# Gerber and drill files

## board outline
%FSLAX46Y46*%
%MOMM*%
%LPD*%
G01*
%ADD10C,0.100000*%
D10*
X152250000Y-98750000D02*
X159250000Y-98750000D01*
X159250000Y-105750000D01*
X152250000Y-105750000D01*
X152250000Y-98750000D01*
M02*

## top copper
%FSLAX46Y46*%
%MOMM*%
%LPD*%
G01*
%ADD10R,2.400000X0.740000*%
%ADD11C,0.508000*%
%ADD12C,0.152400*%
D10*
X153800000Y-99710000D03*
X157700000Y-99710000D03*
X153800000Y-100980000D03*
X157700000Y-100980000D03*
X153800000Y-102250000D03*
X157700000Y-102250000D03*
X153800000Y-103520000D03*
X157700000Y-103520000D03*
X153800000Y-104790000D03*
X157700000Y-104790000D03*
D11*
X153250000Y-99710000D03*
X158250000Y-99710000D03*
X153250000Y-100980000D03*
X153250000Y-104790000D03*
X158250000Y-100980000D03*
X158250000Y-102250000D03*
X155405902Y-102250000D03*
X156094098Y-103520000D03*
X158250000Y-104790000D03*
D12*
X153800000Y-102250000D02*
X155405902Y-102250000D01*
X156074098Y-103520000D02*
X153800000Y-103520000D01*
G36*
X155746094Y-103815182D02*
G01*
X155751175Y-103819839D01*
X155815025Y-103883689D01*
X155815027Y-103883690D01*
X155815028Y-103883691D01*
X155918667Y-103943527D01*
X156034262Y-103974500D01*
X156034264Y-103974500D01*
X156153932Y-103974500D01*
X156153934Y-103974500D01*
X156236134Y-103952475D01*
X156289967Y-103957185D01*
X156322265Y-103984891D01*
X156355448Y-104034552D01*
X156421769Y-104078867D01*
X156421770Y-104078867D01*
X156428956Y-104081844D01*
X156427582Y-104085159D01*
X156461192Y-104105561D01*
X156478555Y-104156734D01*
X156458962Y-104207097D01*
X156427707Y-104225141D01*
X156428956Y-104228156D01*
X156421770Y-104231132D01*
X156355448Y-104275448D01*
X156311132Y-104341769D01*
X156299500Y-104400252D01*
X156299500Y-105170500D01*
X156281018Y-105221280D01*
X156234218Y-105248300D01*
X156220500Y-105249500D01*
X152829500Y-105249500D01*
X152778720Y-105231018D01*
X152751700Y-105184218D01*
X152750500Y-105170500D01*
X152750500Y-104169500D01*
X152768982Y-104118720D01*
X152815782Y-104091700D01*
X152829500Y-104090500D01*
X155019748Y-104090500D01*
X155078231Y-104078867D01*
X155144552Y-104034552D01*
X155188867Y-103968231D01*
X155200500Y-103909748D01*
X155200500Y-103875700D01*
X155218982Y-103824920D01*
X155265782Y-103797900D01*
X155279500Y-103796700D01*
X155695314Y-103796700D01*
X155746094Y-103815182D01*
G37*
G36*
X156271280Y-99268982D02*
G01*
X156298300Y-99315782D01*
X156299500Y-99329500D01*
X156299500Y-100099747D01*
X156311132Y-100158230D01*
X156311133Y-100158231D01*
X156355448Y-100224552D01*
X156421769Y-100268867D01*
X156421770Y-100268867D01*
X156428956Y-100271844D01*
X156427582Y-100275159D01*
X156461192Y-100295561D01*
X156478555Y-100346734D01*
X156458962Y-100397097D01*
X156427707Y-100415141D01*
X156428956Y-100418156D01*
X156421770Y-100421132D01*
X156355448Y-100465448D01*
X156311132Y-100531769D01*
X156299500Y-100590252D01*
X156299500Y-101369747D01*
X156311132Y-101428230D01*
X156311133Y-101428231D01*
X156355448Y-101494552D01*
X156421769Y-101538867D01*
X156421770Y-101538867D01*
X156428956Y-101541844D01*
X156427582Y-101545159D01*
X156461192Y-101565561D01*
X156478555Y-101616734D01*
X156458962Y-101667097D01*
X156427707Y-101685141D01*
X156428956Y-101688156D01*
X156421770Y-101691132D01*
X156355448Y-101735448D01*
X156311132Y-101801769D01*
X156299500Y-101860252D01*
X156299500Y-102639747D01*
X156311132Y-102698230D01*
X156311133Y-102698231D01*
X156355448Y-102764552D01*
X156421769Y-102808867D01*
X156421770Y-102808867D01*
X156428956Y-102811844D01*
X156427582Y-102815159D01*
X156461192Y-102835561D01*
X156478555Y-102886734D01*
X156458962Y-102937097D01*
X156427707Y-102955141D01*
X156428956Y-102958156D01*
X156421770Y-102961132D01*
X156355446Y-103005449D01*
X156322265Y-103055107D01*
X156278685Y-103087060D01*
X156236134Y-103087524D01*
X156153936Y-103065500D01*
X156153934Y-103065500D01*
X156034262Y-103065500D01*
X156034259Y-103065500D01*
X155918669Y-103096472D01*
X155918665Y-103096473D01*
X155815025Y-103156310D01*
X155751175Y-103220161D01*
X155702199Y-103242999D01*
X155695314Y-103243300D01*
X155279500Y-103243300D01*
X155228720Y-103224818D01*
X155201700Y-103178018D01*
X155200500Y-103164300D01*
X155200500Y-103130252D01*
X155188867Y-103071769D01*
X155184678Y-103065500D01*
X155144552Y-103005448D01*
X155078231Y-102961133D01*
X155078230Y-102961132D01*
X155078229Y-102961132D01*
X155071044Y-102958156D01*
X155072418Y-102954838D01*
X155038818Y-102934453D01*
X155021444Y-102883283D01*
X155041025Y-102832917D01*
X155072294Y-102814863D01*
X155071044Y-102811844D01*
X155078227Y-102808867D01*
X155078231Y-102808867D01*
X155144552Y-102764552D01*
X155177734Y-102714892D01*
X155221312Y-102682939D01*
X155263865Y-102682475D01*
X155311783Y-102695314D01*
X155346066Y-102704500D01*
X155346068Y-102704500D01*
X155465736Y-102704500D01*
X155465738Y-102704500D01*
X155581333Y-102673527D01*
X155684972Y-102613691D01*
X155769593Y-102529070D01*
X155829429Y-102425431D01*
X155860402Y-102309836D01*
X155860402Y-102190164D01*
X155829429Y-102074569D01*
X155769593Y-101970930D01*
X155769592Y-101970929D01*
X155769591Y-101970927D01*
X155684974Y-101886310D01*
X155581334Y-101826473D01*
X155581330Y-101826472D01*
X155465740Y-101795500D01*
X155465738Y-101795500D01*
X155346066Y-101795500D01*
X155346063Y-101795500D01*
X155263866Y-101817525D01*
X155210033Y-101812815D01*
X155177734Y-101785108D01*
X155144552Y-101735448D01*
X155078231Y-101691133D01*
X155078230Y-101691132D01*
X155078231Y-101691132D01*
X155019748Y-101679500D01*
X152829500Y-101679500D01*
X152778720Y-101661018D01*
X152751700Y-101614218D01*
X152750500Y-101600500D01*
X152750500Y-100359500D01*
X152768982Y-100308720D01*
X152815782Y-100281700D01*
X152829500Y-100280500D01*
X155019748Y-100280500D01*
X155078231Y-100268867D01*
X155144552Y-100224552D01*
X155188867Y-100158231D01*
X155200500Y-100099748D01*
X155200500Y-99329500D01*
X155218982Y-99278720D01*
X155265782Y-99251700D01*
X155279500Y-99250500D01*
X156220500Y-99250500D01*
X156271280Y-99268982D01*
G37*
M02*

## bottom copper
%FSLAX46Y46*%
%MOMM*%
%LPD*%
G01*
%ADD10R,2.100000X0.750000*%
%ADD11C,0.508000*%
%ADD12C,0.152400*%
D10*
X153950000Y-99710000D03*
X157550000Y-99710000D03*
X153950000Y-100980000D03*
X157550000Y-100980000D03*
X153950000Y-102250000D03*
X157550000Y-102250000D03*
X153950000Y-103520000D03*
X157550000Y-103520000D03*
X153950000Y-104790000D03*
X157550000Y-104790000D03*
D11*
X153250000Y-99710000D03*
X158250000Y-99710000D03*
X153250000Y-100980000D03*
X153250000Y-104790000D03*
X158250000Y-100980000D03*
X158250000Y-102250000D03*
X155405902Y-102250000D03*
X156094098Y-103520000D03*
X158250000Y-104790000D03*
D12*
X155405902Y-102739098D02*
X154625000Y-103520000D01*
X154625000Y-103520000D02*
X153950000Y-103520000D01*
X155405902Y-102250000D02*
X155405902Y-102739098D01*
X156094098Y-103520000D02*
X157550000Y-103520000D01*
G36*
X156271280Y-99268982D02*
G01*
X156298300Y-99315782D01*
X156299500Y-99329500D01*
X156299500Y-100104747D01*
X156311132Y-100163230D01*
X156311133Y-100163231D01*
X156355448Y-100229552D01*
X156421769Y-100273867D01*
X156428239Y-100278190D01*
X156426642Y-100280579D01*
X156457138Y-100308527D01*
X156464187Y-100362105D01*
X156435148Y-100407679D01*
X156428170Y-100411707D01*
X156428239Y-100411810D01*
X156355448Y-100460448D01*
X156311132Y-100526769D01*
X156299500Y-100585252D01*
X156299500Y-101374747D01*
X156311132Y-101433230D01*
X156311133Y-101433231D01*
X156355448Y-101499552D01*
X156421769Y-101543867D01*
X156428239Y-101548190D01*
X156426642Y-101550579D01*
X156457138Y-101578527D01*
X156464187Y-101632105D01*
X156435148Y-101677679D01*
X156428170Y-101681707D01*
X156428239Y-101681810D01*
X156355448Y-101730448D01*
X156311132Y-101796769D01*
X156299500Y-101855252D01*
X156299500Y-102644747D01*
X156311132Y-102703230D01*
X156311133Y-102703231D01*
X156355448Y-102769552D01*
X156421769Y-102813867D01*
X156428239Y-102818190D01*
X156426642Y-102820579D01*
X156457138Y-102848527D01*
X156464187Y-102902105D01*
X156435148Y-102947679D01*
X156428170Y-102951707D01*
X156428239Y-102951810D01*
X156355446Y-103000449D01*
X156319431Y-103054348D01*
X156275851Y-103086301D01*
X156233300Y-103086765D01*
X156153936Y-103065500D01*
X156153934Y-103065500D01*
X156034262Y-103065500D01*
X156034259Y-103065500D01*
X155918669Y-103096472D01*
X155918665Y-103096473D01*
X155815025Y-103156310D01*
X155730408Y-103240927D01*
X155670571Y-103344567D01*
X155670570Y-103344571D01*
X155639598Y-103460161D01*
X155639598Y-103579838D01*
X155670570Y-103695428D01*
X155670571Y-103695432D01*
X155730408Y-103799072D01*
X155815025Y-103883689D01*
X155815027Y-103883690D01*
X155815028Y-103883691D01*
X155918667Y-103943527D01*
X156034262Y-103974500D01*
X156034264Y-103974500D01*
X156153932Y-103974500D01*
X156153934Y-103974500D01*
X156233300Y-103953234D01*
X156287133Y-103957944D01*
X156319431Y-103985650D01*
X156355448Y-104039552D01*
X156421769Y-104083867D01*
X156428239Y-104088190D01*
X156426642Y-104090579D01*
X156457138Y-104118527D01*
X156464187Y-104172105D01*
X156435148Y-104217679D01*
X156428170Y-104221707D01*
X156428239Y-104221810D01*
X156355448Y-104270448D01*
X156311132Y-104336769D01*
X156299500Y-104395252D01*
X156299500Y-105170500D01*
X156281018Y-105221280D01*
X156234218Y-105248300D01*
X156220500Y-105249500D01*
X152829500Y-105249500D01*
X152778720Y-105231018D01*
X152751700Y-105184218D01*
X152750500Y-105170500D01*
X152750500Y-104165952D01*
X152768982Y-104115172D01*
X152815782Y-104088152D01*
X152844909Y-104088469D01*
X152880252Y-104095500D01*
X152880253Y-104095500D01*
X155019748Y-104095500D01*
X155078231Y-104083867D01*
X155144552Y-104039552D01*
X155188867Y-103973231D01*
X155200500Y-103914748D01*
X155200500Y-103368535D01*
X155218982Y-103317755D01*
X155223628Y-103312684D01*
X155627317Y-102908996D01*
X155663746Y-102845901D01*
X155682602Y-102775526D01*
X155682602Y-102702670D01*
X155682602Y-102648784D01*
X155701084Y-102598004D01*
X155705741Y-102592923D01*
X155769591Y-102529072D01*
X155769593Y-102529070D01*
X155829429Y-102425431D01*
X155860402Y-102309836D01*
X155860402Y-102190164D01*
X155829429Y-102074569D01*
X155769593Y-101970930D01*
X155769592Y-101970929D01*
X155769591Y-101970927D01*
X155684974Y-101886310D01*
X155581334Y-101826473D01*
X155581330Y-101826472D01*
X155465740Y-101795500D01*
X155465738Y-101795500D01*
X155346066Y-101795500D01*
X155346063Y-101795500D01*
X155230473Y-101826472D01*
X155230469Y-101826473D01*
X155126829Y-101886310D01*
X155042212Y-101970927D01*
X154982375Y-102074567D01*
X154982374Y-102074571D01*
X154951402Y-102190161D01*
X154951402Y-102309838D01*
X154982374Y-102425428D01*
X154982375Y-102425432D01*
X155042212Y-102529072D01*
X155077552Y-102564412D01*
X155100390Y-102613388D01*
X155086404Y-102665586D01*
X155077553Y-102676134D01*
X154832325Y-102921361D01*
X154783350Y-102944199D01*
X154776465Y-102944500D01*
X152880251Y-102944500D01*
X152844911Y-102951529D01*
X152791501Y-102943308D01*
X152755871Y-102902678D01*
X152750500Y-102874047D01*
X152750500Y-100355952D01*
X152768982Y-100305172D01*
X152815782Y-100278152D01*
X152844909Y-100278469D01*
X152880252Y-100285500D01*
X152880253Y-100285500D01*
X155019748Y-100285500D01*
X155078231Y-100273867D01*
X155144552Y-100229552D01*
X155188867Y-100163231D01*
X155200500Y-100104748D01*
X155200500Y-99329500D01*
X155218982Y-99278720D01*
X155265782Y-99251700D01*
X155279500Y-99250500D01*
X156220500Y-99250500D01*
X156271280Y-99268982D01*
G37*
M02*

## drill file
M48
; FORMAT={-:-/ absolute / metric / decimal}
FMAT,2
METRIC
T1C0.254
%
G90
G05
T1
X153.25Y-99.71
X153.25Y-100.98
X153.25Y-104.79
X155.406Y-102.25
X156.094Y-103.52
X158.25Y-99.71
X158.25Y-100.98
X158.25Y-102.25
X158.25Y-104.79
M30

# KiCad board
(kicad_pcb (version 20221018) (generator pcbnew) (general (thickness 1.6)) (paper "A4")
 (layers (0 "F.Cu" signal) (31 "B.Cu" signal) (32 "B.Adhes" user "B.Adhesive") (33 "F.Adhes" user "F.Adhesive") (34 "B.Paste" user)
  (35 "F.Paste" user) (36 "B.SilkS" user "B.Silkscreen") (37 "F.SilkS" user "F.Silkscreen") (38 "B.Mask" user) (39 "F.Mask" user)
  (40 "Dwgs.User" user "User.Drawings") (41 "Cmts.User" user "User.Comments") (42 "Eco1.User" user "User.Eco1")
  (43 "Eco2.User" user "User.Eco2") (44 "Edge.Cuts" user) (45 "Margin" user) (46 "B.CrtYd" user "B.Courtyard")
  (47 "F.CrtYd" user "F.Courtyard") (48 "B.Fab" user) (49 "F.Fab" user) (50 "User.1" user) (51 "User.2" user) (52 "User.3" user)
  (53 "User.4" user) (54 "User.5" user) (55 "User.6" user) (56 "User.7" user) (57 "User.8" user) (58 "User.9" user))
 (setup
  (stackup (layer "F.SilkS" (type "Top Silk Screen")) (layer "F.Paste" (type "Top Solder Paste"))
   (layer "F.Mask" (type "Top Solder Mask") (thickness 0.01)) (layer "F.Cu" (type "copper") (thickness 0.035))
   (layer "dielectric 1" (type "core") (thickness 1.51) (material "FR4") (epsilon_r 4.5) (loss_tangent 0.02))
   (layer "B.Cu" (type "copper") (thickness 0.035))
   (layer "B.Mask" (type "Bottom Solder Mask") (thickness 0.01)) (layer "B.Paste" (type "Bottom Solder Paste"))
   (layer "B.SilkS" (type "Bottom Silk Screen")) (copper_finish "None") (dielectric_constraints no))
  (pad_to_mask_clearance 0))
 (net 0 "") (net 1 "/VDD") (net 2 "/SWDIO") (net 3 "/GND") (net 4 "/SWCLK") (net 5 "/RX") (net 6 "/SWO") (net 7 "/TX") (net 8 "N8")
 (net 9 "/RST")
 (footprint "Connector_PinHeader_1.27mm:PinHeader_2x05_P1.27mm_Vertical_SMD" (layer "F.Cu") (at 155.75 102.25)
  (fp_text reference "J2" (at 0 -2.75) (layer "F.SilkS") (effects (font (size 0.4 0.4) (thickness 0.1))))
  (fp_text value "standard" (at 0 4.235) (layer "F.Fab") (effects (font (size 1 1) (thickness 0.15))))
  (pad "1" smd rect (at -1.95 -2.54) (size 2.4 0.74) (layers "F.Cu" "F.Paste" "F.Mask") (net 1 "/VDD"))
  (pad "2" smd rect (at 1.95 -2.54) (size 2.4 0.74) (layers "F.Cu" "F.Paste" "F.Mask") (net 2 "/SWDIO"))
  (pad "3" smd rect (at -1.95 -1.27) (size 2.4 0.74) (layers "F.Cu" "F.Paste" "F.Mask") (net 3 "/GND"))
  (pad "4" smd rect (at 1.95 -1.27) (size 2.4 0.74) (layers "F.Cu" "F.Paste" "F.Mask") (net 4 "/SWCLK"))
  (pad "5" smd rect (at -1.95 0) (size 2.4 0.74) (layers "F.Cu" "F.Paste" "F.Mask") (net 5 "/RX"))
  (pad "6" smd rect (at 1.95 0) (size 2.4 0.74) (layers "F.Cu" "F.Paste" "F.Mask") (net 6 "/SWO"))
  (pad "7" smd rect (at -1.95 1.27) (size 2.4 0.74) (layers "F.Cu" "F.Paste" "F.Mask") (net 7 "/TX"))
  (pad "8" smd rect (at 1.95 1.27) (size 2.4 0.74) (layers "F.Cu" "F.Paste" "F.Mask") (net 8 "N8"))
  (pad "9" smd rect (at -1.95 2.54) (size 2.4 0.74) (layers "F.Cu" "F.Paste" "F.Mask") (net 3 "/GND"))
  (pad "10" smd rect (at 1.95 2.54) (size 2.4 0.74) (layers "F.Cu" "F.Paste" "F.Mask") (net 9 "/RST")))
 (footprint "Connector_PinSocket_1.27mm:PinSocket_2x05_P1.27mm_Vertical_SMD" (layer "B.Cu") (at 155.75 102.25 180)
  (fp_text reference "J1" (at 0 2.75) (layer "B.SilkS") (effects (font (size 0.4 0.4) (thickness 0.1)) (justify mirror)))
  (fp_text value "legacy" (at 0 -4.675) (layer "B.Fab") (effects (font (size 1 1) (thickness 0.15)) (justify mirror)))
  (pad "1" smd rect (at 1.8 2.54 180) (size 2.1 0.75) (layers "B.Cu" "B.Paste" "B.Mask") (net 1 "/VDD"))
  (pad "2" smd rect (at -1.8 2.54 180) (size 2.1 0.75) (layers "B.Cu" "B.Paste" "B.Mask") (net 2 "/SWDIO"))
  (pad "3" smd rect (at 1.8 1.27 180) (size 2.1 0.75) (layers "B.Cu" "B.Paste" "B.Mask") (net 3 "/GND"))
  (pad "4" smd rect (at -1.8 1.27 180) (size 2.1 0.75) (layers "B.Cu" "B.Paste" "B.Mask") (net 4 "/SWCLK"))
  (pad "5" smd rect (at 1.8 0 180) (size 2.1 0.75) (layers "B.Cu" "B.Paste" "B.Mask") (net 3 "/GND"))
  (pad "6" smd rect (at -1.8 0 180) (size 2.1 0.75) (layers "B.Cu" "B.Paste" "B.Mask") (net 6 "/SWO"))
  (pad "7" smd rect (at 1.8 -1.27 180) (size 2.1 0.75) (layers "B.Cu" "B.Paste" "B.Mask") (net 5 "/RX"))
  (pad "8" smd rect (at -1.8 -1.27 180) (size 2.1 0.75) (layers "B.Cu" "B.Paste" "B.Mask") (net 7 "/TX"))
  (pad "9" smd rect (at 1.8 -2.54 180) (size 2.1 0.75) (layers "B.Cu" "B.Paste" "B.Mask") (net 3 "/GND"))
  (pad "10" smd rect (at -1.8 -2.54 180) (size 2.1 0.75) (layers "B.Cu" "B.Paste" "B.Mask") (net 9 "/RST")))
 (gr_rect (start 152.25 98.75) (end 159.25 105.75) (stroke (width 0.1) (type solid)) (fill none) (layer "Edge.Cuts"))
 (via (at 153.25 99.71) (size 0.508) (drill 0.254) (layers "F.Cu" "B.Cu") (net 1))
 (via (at 158.25 99.71) (size 0.508) (drill 0.254) (layers "F.Cu" "B.Cu") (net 2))
 (via (at 153.25 100.98) (size 0.508) (drill 0.254) (layers "F.Cu" "B.Cu") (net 3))
 (via (at 153.25 104.79) (size 0.508) (drill 0.254) (layers "F.Cu" "B.Cu") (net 3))
 (via (at 158.25 100.98) (size 0.508) (drill 0.254) (layers "F.Cu" "B.Cu") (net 4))
 (via (at 158.25 102.25) (size 0.508) (drill 0.254) (layers "F.Cu" "B.Cu") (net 6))
 (segment (start 153.8 102.25) (end 155.405902 102.25) (width 0.1524) (layer "F.Cu") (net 5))
 (via (at 155.405902 102.25) (size 0.508) (drill 0.254) (layers "F.Cu" "B.Cu") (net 5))
 (segment (start 155.405902 102.739098) (end 154.625 103.52) (width 0.1524) (layer "B.Cu") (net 5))
 (segment (start 154.625 103.52) (end 153.95 103.52) (width 0.1524) (layer "B.Cu") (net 5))
 (segment (start 155.405902 102.25) (end 155.405902 102.739098) (width 0.1524) (layer "B.Cu") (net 5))
 (segment (start 156.074098 103.52) (end 153.8 103.52) (width 0.1524) (layer "F.Cu") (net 7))
 (via (at 156.094098 103.52) (size 0.508) (drill 0.254) (layers "F.Cu" "B.Cu") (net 7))
 (segment (start 156.094098 103.52) (end 157.55 103.52) (width 0.1524) (layer "B.Cu") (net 7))
 (via (at 158.25 104.79) (size 0.508) (drill 0.254) (layers "F.Cu" "B.Cu") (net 9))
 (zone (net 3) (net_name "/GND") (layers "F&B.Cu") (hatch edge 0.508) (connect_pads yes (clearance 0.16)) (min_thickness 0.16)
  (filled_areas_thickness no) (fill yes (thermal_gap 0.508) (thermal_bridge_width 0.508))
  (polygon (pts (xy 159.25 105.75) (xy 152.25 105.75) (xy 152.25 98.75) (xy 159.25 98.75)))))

